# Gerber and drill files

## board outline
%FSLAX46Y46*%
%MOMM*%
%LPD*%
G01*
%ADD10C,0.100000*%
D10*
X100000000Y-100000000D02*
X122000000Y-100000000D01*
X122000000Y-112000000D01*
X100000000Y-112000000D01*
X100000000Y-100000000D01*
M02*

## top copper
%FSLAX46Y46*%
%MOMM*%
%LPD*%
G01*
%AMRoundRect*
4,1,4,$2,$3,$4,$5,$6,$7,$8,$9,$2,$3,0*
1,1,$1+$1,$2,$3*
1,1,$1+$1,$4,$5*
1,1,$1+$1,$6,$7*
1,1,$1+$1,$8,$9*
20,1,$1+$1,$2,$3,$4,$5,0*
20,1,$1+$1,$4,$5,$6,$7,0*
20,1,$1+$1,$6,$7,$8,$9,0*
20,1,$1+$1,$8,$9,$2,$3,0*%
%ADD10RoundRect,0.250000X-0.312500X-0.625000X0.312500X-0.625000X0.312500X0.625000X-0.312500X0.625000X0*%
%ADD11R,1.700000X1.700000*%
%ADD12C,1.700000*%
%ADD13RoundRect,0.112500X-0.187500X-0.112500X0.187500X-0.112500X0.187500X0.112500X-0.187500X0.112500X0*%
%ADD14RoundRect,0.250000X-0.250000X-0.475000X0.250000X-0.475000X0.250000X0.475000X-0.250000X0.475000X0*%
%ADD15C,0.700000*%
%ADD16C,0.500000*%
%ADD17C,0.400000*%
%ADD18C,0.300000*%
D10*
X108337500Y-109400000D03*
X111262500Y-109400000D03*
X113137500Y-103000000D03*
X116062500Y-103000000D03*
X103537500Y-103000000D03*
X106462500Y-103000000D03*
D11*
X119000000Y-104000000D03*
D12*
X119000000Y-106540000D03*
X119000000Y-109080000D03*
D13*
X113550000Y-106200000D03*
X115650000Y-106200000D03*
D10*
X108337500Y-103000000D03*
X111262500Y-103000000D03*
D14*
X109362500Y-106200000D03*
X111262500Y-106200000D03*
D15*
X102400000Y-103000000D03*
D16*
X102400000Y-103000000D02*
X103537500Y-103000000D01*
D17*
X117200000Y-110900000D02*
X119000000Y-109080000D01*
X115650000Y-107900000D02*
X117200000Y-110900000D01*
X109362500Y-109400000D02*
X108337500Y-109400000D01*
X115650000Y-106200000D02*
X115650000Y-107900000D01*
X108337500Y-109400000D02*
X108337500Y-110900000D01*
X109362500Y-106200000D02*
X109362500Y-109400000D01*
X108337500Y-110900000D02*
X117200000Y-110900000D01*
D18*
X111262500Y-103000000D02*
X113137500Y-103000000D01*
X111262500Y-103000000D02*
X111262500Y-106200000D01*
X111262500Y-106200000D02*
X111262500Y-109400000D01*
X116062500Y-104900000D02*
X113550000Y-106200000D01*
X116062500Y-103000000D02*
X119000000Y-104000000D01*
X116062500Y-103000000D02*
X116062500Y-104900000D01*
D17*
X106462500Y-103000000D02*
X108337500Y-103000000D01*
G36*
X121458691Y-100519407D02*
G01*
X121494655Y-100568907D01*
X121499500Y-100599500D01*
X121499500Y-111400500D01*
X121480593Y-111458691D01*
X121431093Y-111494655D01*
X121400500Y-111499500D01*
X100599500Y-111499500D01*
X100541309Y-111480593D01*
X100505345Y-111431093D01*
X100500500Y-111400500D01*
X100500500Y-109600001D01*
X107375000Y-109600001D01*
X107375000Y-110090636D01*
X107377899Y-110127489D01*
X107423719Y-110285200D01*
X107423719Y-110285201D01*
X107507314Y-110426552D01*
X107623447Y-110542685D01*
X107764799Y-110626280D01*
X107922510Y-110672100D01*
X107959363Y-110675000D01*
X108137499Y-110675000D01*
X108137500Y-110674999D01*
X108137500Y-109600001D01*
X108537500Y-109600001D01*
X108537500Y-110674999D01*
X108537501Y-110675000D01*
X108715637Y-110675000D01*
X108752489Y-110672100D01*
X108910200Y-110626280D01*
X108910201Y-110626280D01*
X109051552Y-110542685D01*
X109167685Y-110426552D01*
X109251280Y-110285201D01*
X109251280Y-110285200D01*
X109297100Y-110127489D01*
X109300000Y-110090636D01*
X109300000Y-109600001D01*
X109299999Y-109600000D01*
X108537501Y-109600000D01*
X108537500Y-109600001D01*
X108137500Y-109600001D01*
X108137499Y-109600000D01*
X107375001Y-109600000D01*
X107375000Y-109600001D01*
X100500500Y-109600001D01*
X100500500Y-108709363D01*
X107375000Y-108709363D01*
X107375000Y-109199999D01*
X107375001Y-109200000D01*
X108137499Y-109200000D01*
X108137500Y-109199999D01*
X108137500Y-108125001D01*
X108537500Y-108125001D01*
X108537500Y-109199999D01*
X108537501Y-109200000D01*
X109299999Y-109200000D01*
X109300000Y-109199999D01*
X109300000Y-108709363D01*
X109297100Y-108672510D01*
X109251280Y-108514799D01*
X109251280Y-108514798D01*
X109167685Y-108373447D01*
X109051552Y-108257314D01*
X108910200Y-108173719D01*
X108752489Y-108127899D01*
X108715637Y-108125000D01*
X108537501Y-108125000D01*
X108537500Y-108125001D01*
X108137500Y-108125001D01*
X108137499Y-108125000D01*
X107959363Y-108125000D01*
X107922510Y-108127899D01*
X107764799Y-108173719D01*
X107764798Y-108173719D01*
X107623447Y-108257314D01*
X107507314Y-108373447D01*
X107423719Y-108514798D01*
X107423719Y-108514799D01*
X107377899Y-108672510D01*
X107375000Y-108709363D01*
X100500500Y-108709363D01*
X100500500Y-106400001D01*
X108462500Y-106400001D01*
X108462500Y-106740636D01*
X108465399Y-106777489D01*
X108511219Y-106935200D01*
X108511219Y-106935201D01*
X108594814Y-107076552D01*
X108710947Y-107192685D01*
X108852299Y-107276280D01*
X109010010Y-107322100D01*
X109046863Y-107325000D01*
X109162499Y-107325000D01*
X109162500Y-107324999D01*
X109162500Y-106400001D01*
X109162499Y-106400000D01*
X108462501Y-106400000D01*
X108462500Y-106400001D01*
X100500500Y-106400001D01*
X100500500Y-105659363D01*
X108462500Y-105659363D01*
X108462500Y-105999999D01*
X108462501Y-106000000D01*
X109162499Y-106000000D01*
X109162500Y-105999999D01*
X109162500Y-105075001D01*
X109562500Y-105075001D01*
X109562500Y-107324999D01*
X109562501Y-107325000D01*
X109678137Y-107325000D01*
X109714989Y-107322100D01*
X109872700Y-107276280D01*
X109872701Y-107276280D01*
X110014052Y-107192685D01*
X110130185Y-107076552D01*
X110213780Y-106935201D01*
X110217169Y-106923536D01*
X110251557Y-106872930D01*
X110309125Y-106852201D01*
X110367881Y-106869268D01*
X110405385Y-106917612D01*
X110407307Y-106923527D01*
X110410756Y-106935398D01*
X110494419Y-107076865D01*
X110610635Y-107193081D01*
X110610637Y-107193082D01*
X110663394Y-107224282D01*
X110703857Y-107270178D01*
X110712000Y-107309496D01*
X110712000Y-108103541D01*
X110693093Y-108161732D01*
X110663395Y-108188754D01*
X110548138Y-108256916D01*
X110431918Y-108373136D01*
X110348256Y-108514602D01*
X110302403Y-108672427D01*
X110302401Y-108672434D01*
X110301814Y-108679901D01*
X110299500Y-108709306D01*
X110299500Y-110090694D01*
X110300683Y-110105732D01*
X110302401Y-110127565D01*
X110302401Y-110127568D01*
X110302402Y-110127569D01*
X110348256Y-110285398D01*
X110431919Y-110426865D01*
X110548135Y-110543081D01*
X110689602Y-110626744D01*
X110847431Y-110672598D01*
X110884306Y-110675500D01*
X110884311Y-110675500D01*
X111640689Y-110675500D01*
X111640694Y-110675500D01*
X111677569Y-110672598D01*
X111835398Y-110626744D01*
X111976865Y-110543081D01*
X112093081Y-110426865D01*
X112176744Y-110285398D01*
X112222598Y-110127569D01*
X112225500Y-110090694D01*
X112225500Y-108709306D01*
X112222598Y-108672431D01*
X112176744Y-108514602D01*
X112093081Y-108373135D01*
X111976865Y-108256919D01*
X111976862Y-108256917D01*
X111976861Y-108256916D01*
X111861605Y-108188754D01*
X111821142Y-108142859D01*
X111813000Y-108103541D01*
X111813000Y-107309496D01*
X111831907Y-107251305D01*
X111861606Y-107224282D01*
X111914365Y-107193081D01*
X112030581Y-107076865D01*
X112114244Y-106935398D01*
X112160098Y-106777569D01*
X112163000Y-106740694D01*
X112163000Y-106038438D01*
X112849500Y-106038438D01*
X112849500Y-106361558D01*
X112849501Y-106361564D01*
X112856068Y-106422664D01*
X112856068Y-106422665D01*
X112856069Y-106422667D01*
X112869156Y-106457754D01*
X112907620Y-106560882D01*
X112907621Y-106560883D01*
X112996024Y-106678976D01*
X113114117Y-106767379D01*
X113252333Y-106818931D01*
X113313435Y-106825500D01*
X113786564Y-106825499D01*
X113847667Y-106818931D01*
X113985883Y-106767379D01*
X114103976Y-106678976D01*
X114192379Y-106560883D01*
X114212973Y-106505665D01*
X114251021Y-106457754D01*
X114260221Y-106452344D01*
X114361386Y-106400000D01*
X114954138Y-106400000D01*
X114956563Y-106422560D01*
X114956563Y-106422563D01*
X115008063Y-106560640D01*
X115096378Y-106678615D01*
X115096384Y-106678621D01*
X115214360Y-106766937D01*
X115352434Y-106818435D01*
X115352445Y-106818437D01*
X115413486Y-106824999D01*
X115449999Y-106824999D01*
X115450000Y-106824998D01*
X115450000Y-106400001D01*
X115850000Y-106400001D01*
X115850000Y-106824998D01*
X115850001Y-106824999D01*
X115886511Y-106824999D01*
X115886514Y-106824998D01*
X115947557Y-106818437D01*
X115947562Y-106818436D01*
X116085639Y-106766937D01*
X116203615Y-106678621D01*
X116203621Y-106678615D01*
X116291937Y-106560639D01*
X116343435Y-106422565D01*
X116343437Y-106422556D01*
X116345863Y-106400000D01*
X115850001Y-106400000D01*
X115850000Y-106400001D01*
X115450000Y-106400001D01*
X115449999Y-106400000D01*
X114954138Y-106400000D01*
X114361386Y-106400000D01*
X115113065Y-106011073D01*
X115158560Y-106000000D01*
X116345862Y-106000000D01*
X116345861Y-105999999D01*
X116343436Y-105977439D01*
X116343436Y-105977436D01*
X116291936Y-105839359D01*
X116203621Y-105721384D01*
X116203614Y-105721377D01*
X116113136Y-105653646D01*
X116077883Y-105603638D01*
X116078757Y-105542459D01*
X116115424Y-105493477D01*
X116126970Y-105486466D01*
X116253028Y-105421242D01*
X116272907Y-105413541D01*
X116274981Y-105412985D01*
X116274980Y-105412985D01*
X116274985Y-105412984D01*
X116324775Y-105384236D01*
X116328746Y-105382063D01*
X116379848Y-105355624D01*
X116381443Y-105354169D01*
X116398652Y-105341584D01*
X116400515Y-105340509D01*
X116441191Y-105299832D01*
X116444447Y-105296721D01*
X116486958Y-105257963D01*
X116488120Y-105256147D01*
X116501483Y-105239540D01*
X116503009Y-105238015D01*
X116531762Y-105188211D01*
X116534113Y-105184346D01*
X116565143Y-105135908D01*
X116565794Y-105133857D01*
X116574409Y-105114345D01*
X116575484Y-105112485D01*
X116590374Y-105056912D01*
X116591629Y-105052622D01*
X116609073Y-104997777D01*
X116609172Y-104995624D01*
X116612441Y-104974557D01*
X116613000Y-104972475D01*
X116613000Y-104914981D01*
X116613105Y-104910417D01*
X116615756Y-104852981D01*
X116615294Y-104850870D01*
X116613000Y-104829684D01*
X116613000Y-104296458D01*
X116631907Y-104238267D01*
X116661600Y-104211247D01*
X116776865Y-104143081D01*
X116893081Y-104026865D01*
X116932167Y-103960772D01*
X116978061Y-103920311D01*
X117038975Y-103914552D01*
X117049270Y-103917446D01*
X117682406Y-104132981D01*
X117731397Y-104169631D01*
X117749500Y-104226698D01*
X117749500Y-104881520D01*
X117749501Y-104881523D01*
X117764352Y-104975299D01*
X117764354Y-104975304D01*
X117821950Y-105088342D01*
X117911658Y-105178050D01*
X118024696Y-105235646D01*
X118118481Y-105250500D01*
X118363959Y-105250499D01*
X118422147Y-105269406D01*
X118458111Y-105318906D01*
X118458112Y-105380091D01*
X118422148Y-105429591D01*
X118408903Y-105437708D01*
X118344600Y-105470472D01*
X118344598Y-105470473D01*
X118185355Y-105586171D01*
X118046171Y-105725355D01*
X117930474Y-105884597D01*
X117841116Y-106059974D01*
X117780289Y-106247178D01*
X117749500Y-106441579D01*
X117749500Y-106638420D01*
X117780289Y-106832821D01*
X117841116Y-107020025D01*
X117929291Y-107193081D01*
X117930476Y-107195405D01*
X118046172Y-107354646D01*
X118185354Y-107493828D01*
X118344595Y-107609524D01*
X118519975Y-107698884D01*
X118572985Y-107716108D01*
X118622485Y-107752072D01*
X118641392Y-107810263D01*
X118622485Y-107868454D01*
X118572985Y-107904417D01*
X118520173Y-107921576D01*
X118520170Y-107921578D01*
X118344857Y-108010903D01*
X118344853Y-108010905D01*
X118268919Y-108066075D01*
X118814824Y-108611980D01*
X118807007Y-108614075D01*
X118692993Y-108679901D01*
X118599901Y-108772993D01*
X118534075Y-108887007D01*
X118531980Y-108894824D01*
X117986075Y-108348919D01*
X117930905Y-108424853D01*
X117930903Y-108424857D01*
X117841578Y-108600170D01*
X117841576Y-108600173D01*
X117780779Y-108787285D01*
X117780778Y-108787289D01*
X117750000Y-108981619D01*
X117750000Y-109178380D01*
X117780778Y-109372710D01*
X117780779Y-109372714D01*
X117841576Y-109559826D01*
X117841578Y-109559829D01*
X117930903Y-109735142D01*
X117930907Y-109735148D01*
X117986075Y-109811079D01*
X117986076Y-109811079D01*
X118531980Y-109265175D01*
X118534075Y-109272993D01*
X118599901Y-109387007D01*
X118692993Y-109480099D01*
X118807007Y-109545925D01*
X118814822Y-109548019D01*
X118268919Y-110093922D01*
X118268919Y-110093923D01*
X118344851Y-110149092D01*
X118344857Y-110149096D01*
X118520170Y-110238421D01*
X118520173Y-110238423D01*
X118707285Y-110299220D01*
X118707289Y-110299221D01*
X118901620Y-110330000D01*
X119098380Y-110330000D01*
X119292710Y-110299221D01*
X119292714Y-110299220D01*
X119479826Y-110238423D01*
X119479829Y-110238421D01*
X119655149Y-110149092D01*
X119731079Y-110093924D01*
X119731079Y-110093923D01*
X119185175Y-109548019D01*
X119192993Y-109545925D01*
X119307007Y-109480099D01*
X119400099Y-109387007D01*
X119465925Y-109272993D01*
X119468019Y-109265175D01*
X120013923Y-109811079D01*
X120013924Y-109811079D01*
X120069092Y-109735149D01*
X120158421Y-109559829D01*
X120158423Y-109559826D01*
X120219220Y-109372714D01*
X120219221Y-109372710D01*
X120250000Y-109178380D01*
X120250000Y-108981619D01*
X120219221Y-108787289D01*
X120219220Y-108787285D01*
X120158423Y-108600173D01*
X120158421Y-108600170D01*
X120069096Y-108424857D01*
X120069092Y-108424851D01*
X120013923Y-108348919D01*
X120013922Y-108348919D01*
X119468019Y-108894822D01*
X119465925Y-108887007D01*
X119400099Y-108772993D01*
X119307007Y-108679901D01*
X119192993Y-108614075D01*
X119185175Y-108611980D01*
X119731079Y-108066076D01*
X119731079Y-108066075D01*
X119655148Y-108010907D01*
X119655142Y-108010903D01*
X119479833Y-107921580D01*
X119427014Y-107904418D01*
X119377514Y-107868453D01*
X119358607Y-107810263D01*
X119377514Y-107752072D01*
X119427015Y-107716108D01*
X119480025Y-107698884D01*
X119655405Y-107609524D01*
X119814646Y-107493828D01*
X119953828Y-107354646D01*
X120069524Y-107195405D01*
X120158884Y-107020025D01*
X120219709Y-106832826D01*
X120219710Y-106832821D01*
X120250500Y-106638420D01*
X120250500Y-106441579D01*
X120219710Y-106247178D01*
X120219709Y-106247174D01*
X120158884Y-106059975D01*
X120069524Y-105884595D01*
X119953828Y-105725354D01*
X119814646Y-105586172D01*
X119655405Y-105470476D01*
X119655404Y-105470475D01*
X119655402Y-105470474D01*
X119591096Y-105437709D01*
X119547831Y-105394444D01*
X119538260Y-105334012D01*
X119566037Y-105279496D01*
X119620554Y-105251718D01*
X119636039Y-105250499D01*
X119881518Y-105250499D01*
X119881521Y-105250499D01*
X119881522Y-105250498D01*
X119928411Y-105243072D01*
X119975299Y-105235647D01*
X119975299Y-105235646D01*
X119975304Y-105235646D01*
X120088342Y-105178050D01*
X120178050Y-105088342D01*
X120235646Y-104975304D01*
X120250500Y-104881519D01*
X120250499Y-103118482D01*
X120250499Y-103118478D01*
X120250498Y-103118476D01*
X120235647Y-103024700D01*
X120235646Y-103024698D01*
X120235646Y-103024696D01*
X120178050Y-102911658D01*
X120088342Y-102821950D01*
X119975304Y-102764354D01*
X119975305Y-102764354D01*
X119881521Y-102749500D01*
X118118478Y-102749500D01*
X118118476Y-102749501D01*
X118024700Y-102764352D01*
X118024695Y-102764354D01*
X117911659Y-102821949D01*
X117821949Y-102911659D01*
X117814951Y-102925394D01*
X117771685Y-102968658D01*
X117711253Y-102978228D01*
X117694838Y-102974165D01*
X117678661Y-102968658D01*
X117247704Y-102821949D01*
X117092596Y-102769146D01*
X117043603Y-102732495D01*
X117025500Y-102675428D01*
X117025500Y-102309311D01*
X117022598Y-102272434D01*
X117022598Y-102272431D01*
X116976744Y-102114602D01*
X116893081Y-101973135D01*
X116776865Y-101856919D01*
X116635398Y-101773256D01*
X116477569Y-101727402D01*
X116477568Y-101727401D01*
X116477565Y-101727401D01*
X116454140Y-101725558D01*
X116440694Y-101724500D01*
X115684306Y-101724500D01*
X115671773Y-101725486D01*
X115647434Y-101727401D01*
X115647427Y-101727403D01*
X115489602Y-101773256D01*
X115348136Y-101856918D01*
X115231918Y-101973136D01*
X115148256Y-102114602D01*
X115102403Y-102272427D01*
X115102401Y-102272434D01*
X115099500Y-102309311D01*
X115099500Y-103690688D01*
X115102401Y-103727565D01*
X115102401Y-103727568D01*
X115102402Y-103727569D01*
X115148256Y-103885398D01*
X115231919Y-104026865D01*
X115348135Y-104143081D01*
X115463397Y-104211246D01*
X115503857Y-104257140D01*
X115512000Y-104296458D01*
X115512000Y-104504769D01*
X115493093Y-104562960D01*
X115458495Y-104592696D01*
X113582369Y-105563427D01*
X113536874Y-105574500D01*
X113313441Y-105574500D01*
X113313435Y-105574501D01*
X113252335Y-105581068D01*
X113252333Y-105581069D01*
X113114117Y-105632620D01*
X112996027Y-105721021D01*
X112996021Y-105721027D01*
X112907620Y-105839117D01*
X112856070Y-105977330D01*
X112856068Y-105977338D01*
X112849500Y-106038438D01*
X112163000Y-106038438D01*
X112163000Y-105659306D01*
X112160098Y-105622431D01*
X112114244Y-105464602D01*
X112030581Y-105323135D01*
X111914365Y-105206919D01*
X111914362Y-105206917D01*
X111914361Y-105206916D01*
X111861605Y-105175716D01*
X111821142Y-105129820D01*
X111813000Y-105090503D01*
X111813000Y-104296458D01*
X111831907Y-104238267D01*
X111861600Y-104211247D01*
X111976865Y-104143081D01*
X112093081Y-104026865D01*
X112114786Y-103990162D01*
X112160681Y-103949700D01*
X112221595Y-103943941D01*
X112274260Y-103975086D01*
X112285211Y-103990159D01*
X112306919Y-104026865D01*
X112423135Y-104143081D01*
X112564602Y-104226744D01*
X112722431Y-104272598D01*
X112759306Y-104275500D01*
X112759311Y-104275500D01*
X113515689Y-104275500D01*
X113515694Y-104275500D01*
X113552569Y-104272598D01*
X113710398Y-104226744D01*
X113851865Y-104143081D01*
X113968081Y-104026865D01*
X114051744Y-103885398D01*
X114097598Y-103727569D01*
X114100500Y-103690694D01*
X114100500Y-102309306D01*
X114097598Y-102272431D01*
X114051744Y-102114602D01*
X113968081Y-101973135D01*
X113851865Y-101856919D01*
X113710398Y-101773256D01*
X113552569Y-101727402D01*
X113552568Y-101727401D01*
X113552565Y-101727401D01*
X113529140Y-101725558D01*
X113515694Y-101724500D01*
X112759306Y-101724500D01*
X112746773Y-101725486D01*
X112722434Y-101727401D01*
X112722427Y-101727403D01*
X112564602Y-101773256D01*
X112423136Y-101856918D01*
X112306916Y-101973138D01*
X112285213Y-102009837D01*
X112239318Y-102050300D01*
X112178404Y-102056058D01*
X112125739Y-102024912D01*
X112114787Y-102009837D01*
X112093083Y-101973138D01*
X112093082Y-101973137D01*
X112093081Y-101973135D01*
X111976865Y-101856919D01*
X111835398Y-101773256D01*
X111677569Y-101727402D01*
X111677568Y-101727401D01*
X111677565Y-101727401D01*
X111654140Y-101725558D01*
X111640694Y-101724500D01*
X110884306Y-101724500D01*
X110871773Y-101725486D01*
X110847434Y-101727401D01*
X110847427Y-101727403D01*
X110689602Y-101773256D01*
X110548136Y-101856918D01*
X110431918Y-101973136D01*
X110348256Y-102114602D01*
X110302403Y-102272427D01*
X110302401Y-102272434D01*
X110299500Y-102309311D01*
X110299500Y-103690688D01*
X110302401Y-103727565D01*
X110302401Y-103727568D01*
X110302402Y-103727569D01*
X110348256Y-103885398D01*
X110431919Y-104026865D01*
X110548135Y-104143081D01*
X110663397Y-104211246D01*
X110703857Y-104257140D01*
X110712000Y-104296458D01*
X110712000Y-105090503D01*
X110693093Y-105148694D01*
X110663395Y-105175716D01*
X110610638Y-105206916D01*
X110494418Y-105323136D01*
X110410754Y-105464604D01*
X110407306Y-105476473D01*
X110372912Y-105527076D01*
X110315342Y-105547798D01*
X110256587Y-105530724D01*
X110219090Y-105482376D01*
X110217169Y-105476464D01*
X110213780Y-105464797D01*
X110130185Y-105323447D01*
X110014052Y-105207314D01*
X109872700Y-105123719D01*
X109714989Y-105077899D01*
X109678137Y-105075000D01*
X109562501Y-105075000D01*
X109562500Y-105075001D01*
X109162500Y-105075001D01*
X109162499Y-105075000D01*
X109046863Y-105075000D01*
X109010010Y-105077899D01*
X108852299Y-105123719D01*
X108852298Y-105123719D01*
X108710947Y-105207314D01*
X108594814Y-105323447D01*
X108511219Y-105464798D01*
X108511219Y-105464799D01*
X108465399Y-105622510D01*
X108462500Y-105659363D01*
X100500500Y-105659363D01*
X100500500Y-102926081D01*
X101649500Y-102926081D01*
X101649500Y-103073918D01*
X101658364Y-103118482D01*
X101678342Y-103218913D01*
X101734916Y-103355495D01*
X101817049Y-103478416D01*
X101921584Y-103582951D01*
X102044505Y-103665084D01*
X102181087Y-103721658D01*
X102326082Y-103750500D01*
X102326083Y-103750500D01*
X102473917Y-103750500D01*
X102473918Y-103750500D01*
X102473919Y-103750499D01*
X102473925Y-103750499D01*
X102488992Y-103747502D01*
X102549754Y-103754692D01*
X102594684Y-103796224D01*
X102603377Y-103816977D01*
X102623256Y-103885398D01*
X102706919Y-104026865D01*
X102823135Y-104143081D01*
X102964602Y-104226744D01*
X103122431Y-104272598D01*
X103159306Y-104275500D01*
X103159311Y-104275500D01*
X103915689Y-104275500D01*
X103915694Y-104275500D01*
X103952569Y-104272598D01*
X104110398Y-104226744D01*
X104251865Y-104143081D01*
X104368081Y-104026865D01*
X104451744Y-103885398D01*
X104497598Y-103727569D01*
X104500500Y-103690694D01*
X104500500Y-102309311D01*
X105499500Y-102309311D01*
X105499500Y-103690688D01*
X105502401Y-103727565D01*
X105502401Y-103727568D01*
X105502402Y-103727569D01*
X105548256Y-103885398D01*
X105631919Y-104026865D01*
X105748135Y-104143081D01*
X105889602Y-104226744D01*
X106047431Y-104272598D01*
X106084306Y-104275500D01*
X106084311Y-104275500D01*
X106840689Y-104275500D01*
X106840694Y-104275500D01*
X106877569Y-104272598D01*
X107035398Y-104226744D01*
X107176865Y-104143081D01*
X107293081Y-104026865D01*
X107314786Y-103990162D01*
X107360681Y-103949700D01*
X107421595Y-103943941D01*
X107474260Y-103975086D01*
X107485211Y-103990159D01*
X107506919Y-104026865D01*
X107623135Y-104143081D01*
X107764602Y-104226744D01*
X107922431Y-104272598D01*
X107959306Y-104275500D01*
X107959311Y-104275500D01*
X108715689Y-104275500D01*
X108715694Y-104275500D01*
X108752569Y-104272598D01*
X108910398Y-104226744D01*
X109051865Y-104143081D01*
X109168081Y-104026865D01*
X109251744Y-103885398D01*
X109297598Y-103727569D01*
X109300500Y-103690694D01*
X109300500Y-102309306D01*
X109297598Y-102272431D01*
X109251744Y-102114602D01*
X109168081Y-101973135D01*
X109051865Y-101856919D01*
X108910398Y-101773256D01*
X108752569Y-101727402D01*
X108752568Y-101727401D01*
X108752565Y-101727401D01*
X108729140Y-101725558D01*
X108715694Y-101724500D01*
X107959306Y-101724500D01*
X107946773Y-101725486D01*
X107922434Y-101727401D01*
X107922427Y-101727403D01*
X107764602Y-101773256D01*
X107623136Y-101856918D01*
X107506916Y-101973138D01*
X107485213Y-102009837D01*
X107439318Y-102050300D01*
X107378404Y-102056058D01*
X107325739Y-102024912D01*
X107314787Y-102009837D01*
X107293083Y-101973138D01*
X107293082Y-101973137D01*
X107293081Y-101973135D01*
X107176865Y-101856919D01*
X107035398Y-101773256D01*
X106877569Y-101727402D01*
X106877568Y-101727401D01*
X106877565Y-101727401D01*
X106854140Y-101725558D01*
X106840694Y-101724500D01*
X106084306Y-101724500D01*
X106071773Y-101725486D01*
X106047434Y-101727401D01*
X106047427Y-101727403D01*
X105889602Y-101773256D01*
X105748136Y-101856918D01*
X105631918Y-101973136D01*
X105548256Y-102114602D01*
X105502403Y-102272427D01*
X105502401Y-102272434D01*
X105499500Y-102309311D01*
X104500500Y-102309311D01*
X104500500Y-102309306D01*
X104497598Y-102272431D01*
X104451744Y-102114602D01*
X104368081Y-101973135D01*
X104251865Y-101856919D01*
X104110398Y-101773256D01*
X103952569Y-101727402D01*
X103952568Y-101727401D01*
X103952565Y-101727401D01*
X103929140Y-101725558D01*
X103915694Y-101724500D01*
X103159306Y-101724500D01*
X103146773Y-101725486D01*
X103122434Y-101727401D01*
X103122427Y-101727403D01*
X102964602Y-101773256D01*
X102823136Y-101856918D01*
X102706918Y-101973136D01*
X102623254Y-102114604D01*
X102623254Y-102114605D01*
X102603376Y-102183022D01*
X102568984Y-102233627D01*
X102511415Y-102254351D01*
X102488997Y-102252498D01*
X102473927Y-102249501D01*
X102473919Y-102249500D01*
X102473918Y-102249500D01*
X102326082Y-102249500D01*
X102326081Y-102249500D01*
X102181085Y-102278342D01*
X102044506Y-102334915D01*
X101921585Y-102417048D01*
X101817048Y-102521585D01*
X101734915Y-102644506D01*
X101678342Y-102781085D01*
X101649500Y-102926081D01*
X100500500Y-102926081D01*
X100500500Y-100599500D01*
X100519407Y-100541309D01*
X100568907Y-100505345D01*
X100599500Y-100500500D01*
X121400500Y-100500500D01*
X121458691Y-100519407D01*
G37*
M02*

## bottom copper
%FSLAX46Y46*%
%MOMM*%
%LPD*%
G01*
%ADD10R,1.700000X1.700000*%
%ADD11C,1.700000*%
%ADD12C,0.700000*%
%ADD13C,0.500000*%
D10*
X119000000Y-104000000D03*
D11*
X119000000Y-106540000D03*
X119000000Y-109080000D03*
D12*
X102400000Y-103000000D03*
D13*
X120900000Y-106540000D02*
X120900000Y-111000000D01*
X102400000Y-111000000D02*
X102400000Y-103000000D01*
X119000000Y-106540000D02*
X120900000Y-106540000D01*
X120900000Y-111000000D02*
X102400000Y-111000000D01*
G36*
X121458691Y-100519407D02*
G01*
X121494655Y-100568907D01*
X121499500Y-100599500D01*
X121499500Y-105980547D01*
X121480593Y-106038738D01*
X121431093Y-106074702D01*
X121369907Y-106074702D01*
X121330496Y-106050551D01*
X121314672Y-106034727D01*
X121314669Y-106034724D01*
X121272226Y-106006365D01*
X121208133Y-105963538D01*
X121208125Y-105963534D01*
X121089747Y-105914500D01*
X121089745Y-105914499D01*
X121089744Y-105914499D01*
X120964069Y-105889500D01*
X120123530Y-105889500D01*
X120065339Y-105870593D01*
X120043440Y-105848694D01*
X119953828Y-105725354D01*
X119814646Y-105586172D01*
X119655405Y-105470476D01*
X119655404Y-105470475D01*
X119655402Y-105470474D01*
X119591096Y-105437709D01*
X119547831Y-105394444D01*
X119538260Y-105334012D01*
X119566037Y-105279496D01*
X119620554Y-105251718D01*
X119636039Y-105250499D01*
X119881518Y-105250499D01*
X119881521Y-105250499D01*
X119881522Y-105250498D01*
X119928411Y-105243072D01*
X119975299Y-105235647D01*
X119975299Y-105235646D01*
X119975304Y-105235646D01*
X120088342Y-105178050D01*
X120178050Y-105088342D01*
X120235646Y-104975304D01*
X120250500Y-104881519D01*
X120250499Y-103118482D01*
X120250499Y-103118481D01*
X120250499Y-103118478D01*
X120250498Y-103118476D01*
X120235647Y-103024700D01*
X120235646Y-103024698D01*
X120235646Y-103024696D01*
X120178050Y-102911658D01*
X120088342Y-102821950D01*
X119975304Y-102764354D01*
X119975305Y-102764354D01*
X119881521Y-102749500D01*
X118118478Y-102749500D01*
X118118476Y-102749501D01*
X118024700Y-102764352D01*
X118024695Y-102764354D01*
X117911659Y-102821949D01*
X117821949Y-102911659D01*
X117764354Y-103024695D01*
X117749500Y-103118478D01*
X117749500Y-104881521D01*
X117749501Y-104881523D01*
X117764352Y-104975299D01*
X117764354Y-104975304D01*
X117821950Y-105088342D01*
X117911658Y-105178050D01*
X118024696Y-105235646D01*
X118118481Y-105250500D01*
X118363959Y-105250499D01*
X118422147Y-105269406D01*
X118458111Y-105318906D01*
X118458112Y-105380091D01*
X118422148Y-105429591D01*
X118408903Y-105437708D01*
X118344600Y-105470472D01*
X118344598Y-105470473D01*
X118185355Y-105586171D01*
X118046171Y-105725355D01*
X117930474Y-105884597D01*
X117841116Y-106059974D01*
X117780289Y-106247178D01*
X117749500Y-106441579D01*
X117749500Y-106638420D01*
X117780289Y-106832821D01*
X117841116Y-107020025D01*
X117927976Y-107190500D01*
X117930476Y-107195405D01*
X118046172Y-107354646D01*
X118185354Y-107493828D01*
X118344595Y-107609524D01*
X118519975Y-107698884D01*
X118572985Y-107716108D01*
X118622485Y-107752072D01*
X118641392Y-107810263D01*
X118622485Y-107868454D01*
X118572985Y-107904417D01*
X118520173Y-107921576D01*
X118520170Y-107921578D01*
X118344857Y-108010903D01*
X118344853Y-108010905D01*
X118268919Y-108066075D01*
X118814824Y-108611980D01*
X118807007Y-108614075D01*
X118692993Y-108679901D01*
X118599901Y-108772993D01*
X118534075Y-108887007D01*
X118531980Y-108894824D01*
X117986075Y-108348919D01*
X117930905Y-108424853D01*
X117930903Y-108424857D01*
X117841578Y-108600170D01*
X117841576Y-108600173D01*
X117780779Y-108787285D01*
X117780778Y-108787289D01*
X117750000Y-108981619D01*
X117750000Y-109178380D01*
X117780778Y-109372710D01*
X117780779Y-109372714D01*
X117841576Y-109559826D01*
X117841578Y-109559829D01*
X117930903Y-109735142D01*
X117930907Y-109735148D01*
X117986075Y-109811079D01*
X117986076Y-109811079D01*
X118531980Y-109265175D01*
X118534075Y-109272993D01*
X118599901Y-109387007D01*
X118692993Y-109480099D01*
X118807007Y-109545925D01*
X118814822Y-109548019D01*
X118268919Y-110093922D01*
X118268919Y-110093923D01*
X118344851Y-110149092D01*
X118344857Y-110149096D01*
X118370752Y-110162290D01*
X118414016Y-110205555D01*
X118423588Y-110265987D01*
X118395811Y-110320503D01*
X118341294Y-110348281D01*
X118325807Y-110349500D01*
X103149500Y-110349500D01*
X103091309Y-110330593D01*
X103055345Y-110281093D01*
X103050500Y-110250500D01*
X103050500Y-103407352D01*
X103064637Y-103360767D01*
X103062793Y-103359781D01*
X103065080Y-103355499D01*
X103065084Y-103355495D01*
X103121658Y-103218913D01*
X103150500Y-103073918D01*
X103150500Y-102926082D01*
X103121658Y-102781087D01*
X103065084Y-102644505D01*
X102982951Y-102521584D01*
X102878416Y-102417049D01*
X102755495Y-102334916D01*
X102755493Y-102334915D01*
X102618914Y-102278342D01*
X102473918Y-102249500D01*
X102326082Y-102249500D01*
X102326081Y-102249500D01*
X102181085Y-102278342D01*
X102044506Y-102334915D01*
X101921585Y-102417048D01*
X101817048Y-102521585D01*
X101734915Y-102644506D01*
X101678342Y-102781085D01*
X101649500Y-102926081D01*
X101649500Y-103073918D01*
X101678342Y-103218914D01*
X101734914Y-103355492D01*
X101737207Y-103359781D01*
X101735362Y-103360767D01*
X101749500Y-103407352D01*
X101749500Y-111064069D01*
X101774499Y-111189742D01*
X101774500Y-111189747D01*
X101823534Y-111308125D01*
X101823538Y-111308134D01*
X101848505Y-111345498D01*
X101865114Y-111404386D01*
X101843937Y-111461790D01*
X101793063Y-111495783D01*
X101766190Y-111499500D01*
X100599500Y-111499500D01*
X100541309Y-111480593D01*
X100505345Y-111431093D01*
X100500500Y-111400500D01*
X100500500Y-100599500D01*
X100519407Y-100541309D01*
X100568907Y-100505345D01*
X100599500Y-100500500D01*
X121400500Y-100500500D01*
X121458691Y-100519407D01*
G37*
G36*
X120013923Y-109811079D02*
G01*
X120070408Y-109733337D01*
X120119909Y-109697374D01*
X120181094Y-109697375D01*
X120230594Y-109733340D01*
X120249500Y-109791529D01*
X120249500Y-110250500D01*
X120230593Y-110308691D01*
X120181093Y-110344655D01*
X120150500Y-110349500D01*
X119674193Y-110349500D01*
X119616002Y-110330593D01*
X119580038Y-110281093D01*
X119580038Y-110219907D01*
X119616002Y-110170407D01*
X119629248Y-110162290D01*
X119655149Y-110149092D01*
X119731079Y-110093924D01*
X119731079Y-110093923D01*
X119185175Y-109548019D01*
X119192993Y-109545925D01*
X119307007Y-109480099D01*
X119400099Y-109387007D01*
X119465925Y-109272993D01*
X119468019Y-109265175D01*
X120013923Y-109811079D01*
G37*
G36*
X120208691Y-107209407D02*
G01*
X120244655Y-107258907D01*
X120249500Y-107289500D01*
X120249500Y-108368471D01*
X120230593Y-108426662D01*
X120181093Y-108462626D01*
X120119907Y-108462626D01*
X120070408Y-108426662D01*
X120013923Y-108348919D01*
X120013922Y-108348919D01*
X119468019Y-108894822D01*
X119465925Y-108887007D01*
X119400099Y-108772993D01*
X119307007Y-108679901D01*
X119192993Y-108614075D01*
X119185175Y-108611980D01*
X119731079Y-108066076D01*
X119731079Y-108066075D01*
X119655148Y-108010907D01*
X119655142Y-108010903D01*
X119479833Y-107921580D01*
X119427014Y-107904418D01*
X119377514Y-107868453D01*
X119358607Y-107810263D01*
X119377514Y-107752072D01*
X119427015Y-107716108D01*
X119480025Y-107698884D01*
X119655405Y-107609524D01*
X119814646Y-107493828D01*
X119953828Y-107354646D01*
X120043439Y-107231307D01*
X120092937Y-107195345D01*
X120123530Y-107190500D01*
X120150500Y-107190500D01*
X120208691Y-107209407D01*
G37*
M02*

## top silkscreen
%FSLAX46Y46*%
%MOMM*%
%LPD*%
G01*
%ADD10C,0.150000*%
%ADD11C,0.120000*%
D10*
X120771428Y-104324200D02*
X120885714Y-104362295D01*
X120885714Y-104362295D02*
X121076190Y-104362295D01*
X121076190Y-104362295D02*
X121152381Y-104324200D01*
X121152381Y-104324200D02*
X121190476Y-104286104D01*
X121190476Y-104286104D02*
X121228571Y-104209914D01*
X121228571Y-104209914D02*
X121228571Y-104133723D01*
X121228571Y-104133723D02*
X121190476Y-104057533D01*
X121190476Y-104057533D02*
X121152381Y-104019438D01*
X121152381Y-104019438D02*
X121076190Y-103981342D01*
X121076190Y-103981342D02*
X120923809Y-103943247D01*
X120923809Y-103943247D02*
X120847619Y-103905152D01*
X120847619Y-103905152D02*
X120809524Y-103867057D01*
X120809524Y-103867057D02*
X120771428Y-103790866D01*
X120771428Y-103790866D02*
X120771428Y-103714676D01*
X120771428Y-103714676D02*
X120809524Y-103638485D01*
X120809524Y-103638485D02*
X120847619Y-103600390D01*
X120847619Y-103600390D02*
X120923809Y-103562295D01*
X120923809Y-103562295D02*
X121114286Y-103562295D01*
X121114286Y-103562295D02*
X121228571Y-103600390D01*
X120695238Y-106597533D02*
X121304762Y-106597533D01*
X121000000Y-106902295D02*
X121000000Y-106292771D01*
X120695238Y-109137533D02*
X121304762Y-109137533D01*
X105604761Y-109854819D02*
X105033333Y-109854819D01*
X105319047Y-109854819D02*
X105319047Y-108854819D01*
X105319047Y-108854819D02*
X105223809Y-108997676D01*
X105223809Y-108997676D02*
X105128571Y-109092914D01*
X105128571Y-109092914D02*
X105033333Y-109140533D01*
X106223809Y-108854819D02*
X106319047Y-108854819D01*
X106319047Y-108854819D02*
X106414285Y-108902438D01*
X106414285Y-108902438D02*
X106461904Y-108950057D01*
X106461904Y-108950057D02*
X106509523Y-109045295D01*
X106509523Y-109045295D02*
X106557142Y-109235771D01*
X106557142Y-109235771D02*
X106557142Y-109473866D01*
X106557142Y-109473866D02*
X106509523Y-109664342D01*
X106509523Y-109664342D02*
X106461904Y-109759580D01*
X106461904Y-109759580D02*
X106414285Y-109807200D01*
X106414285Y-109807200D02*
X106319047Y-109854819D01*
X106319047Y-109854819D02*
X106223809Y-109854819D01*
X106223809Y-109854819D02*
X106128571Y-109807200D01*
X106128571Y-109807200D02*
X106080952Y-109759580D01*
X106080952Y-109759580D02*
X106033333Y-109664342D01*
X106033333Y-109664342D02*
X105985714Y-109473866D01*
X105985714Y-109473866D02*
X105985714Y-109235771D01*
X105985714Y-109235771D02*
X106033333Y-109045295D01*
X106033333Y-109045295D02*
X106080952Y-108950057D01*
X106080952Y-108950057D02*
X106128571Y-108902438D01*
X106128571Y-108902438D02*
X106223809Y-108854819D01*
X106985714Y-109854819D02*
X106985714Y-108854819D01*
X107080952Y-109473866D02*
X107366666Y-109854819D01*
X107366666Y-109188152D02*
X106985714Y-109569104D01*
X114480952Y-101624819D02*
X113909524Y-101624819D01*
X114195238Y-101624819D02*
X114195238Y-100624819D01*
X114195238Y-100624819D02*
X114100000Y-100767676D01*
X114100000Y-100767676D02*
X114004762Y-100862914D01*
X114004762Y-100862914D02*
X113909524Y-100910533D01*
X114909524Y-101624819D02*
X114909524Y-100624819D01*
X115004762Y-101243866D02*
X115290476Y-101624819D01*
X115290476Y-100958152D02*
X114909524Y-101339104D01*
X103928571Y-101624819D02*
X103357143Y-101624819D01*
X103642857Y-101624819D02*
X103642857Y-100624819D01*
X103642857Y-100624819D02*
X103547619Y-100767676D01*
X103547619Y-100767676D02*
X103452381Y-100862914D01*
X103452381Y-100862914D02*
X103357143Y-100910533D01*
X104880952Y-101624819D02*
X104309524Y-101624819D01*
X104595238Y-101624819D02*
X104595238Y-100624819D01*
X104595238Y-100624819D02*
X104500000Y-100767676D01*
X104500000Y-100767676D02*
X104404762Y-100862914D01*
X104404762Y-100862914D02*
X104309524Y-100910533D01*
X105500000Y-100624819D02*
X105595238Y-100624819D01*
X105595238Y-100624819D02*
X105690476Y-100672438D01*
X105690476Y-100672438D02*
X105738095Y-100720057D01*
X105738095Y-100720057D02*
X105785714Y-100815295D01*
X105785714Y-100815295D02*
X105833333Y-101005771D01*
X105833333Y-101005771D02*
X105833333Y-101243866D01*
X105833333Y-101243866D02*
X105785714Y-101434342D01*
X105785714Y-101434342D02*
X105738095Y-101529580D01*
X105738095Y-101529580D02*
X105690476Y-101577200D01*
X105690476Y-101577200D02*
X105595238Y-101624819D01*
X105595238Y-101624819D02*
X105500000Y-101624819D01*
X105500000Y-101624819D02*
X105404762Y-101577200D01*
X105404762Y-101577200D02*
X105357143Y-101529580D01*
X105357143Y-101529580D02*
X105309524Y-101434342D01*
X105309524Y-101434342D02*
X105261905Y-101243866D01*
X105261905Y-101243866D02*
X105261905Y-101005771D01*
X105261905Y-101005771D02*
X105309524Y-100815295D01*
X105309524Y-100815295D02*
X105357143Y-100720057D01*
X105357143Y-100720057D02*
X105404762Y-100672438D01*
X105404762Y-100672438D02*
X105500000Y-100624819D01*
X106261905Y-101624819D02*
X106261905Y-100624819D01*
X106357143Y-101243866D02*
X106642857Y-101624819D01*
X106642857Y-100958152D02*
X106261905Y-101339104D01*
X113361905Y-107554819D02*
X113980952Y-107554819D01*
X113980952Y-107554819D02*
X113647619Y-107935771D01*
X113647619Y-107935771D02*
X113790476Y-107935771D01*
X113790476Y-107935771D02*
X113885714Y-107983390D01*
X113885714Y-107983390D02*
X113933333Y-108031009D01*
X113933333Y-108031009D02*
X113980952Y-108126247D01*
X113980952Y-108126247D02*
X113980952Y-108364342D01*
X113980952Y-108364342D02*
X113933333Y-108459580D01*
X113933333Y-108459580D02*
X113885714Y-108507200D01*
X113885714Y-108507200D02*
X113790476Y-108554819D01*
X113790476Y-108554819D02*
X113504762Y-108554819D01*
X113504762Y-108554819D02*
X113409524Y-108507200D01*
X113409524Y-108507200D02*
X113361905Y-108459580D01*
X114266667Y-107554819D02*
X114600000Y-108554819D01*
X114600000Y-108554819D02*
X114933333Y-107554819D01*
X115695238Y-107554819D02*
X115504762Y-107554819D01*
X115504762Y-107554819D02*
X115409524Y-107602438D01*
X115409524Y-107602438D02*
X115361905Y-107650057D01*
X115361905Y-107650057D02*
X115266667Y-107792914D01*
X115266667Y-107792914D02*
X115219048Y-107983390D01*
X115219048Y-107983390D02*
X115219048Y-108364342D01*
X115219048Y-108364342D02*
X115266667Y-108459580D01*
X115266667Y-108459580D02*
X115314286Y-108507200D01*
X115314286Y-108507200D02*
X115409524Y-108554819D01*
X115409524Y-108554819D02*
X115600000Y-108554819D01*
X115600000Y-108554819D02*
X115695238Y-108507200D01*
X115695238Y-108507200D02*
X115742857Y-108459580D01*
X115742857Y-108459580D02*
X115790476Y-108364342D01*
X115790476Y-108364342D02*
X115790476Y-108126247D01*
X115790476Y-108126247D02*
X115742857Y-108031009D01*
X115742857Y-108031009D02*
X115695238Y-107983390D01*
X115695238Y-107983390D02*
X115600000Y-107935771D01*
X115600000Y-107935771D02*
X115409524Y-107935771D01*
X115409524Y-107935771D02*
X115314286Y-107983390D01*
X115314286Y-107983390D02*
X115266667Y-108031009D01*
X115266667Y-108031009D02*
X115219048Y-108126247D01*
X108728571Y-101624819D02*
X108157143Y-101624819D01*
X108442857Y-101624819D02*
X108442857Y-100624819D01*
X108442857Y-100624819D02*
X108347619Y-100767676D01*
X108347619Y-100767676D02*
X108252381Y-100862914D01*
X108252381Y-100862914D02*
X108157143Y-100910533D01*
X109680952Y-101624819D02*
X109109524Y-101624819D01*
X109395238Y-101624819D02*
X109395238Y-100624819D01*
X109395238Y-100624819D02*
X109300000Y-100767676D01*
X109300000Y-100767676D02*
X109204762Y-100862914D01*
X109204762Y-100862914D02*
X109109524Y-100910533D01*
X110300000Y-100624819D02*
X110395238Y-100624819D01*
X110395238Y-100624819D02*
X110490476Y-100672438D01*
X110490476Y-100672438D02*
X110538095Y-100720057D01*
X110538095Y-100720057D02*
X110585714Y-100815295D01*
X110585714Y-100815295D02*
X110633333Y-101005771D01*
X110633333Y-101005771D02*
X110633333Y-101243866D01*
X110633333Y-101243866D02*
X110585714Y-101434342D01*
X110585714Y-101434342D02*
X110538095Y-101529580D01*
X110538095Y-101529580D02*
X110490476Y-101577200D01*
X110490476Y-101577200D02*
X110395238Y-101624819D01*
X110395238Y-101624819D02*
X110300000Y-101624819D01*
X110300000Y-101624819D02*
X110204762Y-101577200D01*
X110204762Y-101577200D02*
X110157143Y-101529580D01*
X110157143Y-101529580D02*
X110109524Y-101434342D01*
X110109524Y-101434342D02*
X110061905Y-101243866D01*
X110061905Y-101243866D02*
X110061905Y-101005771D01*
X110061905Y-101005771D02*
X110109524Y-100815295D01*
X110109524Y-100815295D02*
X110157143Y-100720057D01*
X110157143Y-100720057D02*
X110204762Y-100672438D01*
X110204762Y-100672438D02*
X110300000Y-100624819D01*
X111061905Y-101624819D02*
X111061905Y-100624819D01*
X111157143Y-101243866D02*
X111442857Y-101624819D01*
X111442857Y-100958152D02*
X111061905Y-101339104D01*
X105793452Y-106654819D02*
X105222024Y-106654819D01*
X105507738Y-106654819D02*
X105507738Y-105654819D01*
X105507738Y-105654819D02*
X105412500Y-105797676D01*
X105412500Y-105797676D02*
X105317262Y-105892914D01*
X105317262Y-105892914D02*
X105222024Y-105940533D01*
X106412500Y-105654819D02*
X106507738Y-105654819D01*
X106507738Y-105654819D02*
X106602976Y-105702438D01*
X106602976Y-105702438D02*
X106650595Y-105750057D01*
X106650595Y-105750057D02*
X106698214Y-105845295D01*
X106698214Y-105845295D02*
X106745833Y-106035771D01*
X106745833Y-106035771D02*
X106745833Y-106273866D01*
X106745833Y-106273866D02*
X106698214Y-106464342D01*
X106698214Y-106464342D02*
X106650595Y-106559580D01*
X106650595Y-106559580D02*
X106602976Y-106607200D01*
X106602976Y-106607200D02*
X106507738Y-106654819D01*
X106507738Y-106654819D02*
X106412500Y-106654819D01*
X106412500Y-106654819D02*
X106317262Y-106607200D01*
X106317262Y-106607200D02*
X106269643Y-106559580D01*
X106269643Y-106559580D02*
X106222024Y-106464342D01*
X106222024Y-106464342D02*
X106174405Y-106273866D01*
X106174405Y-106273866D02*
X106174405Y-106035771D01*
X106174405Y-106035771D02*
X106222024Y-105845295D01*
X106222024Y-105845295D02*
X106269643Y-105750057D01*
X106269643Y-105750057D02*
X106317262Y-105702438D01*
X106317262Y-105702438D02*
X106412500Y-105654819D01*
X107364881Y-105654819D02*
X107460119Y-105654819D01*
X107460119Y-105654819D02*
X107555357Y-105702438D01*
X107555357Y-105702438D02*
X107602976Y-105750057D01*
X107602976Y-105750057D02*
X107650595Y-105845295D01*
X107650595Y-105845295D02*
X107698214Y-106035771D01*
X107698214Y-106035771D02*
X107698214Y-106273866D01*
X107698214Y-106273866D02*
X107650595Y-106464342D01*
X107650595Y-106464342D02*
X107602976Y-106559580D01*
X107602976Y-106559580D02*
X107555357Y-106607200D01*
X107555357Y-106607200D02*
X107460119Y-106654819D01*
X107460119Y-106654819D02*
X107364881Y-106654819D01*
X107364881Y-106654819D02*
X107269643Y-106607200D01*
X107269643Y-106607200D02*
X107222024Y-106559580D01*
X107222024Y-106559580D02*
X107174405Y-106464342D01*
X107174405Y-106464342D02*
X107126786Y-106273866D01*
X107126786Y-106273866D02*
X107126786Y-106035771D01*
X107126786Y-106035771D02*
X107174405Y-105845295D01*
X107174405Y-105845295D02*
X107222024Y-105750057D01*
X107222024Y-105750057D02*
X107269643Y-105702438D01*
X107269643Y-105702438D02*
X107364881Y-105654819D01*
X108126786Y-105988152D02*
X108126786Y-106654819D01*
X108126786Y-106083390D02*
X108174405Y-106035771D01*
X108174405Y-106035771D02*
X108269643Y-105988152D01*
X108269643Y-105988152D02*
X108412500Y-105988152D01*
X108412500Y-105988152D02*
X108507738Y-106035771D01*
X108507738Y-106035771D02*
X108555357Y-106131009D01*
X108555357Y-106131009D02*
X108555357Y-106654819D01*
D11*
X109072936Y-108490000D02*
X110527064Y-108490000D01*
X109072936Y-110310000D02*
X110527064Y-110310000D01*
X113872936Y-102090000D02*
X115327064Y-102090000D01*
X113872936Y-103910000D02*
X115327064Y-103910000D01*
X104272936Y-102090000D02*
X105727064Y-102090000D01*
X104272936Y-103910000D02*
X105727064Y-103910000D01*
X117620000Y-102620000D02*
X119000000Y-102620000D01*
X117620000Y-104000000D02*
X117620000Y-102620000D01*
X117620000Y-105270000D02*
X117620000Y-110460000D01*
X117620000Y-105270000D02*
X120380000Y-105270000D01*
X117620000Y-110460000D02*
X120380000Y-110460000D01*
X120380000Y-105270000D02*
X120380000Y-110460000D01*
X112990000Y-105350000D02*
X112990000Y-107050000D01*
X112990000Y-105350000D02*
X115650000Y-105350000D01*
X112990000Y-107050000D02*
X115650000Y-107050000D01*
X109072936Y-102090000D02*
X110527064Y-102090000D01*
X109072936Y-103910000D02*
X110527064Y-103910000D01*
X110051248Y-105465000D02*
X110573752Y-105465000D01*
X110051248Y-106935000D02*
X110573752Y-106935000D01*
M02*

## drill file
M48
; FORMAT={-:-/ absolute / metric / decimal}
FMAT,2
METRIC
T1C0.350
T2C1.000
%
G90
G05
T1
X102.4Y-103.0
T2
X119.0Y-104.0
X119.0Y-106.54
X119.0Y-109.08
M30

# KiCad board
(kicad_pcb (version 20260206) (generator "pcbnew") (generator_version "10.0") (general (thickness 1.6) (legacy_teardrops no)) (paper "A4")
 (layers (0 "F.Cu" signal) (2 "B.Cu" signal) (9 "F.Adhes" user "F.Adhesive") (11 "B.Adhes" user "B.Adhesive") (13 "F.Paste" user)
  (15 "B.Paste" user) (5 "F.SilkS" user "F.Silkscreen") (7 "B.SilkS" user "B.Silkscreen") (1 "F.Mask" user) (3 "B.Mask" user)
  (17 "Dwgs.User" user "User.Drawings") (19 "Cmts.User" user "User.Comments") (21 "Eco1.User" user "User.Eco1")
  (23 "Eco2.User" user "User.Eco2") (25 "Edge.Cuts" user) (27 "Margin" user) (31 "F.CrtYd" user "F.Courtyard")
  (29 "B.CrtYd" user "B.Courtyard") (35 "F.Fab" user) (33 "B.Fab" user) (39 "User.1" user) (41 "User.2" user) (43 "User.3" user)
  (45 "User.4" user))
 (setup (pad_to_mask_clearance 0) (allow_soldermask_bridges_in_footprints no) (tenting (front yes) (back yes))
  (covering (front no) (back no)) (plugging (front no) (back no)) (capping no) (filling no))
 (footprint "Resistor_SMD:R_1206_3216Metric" (layer "F.Cu") (at 109.8 109.4)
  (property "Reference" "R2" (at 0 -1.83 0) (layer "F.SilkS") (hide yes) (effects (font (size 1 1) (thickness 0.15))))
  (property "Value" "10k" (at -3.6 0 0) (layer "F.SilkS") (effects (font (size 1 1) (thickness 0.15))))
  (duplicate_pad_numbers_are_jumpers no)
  (fp_line (start -0.727064 -0.91) (end 0.727064 -0.91) (stroke (width 0.12) (type solid)) (layer "F.SilkS"))
  (fp_line (start -0.727064 0.91) (end 0.727064 0.91) (stroke (width 0.12) (type solid)) (layer "F.SilkS"))
  (pad "1" smd roundrect (at -1.4625 0) (size 1.125 1.75) (layers "F.Cu" "F.Mask" "F.Paste") (roundrect_rratio 0.222222) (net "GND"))
  (pad "2" smd roundrect (at 1.4625 0) (size 1.125 1.75) (layers "F.Cu" "F.Mask" "F.Paste") (roundrect_rratio 0.222222) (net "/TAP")))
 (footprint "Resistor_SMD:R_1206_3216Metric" (layer "F.Cu") (at 114.6 103)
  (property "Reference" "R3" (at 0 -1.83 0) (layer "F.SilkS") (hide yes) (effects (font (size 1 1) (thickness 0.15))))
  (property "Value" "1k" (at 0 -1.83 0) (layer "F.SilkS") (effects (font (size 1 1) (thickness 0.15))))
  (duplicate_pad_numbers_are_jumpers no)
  (fp_line (start -0.727064 -0.91) (end 0.727064 -0.91) (stroke (width 0.12) (type solid)) (layer "F.SilkS"))
  (fp_line (start -0.727064 0.91) (end 0.727064 0.91) (stroke (width 0.12) (type solid)) (layer "F.SilkS"))
  (pad "1" smd roundrect (at -1.4625 0) (size 1.125 1.75) (layers "F.Cu" "F.Mask" "F.Paste") (roundrect_rratio 0.222222) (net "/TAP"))
  (pad "2" smd roundrect (at 1.4625 0) (size 1.125 1.75) (layers "F.Cu" "F.Mask" "F.Paste") (roundrect_rratio 0.222222) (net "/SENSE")))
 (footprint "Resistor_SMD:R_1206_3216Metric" (layer "F.Cu") (at 105 103)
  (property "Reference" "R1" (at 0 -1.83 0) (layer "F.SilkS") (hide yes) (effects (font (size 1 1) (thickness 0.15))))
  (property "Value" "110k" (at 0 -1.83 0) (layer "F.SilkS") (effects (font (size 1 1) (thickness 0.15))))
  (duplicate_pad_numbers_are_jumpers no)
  (fp_line (start -0.727064 -0.91) (end 0.727064 -0.91) (stroke (width 0.12) (type solid)) (layer "F.SilkS"))
  (fp_line (start -0.727064 0.91) (end 0.727064 0.91) (stroke (width 0.12) (type solid)) (layer "F.SilkS"))
  (pad "1" smd roundrect (at -1.4625 0) (size 1.125 1.75) (layers "F.Cu" "F.Mask" "F.Paste") (roundrect_rratio 0.222222) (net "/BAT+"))
  (pad "2" smd roundrect (at 1.4625 0) (size 1.125 1.75) (layers "F.Cu" "F.Mask" "F.Paste") (roundrect_rratio 0.222222) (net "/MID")))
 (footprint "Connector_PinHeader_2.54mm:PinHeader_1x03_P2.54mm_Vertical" (layer "F.Cu") (at 119 104)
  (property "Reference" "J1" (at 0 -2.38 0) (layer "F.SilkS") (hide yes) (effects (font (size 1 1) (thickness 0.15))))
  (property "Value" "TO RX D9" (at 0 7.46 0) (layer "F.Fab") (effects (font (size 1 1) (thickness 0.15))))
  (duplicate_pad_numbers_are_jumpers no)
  (fp_line (start -1.38 -1.38) (end 0 -1.38) (stroke (width 0.12) (type solid)) (layer "F.SilkS"))
  (fp_line (start -1.38 0) (end -1.38 -1.38) (stroke (width 0.12) (type solid)) (layer "F.SilkS"))
  (fp_line (start -1.38 1.27) (end -1.38 6.46) (stroke (width 0.12) (type solid)) (layer "F.SilkS"))
  (fp_line (start -1.38 1.27) (end 1.38 1.27) (stroke (width 0.12) (type solid)) (layer "F.SilkS"))
  (fp_line (start -1.38 6.46) (end 1.38 6.46) (stroke (width 0.12) (type solid)) (layer "F.SilkS"))
  (fp_line (start 1.38 1.27) (end 1.38 6.46) (stroke (width 0.12) (type solid)) (layer "F.SilkS"))
  (pad "1" thru_hole rect (at 0 0) (size 1.7 1.7) (drill 1) (layers "*.Cu" "*.Mask") (remove_unused_layers no) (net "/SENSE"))
  (pad "2" thru_hole circle (at 0 2.54) (size 1.7 1.7) (drill 1) (layers "*.Cu" "*.Mask") (remove_unused_layers no) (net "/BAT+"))
  (pad "3" thru_hole circle (at 0 5.08) (size 1.7 1.7) (drill 1) (layers "*.Cu" "*.Mask") (remove_unused_layers no) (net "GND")))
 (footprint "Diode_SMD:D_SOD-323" (layer "F.Cu") (at 114.6 106.2)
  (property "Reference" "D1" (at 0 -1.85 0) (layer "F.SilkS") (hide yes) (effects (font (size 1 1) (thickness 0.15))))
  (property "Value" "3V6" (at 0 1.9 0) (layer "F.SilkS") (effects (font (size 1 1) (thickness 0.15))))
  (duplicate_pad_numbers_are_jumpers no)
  (fp_line (start -1.61 -0.85) (end -1.61 0.85) (stroke (width 0.12) (type solid)) (layer "F.SilkS"))
  (fp_line (start -1.61 -0.85) (end 1.05 -0.85) (stroke (width 0.12) (type solid)) (layer "F.SilkS"))
  (fp_line (start -1.61 0.85) (end 1.05 0.85) (stroke (width 0.12) (type solid)) (layer "F.SilkS"))
  (pad "1" smd roundrect (at -1.05 0) (size 0.6 0.45) (layers "F.Cu" "F.Mask" "F.Paste") (roundrect_rratio 0.25) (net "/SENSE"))
  (pad "2" smd roundrect (at 1.05 0) (size 0.6 0.45) (layers "F.Cu" "F.Mask" "F.Paste") (roundrect_rratio 0.25) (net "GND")))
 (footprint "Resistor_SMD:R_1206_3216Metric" (layer "F.Cu") (at 109.8 103)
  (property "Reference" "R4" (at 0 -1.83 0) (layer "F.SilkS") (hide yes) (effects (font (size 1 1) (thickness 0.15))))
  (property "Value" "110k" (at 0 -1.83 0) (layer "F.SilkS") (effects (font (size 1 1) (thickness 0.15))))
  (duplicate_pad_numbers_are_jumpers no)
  (fp_line (start -0.727064 -0.91) (end 0.727064 -0.91) (stroke (width 0.12) (type solid)) (layer "F.SilkS"))
  (fp_line (start -0.727064 0.91) (end 0.727064 0.91) (stroke (width 0.12) (type solid)) (layer "F.SilkS"))
  (pad "1" smd roundrect (at -1.4625 0) (size 1.125 1.75) (layers "F.Cu" "F.Mask" "F.Paste") (roundrect_rratio 0.222222) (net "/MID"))
  (pad "2" smd roundrect (at 1.4625 0) (size 1.125 1.75) (layers "F.Cu" "F.Mask" "F.Paste") (roundrect_rratio 0.222222) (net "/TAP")))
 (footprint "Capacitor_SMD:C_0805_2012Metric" (layer "F.Cu") (at 110.3125 106.2)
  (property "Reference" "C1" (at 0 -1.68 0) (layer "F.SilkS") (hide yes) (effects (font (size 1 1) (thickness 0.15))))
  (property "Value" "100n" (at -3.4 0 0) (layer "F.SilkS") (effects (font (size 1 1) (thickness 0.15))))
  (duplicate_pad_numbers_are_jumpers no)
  (fp_line (start -0.261252 -0.735) (end 0.261252 -0.735) (stroke (width 0.12) (type solid)) (layer "F.SilkS"))
  (fp_line (start -0.261252 0.735) (end 0.261252 0.735) (stroke (width 0.12) (type solid)) (layer "F.SilkS"))
  (pad "1" smd roundrect (at -0.95 0) (size 1 1.45) (layers "F.Cu" "F.Mask" "F.Paste") (roundrect_rratio 0.25) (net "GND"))
  (pad "2" smd roundrect (at 0.95 0) (size 1 1.45) (layers "F.Cu" "F.Mask" "F.Paste") (roundrect_rratio 0.25) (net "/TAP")))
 (gr_rect (start 100 100) (end 122 112) (stroke (width 0.1) (type solid)) (fill no) (layer "Edge.Cuts"))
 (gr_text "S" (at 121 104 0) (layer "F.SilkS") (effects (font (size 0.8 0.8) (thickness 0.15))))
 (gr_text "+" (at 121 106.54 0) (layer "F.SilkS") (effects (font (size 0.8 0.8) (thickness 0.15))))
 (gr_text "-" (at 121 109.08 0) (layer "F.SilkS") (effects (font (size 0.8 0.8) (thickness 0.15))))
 (segment (start 102.4 103) (end 103.5375 103) (width 0.5) (layer "F.Cu") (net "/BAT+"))
 (via (at 102.4 103) (size 0.7) (drill 0.35) (layers "F.Cu" "B.Cu") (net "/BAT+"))
 (segment (start 120.9 106.54) (end 120.9 111) (width 0.5) (layer "B.Cu") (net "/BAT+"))
 (segment (start 102.4 111) (end 102.4 103) (width 0.5) (layer "B.Cu") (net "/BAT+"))
 (segment (start 119 106.54) (end 120.9 106.54) (width 0.5) (layer "B.Cu") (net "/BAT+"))
 (segment (start 120.9 111) (end 102.4 111) (width 0.5) (layer "B.Cu") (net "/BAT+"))
 (segment (start 117.2 110.9) (end 119 109.08) (width 0.4) (layer "F.Cu") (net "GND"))
 (segment (start 115.65 107.9) (end 117.2 110.9) (width 0.4) (layer "F.Cu") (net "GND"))
 (segment (start 109.3625 109.4) (end 108.3375 109.4) (width 0.4) (layer "F.Cu") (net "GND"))
 (segment (start 115.65 106.2) (end 115.65 107.9) (width 0.4) (layer "F.Cu") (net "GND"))
 (segment (start 108.3375 109.4) (end 108.3375 110.9) (width 0.4) (layer "F.Cu") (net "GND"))
 (segment (start 109.3625 106.2) (end 109.3625 109.4) (width 0.4) (layer "F.Cu") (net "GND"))
 (segment (start 108.3375 110.9) (end 117.2 110.9) (width 0.4) (layer "F.Cu") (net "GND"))
 (segment (start 111.2625 103) (end 113.1375 103) (width 0.3) (layer "F.Cu") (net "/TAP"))
 (segment (start 111.2625 103) (end 111.2625 106.2) (width 0.3) (layer "F.Cu") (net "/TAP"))
 (segment (start 111.2625 106.2) (end 111.2625 109.4) (width 0.3) (layer "F.Cu") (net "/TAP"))
 (segment (start 116.0625 104.9) (end 113.55 106.2) (width 0.3) (layer "F.Cu") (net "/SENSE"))
 (segment (start 116.0625 103) (end 119 104) (width 0.3) (layer "F.Cu") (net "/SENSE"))
 (segment (start 116.0625 103) (end 116.0625 104.9) (width 0.3) (layer "F.Cu") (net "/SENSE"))
 (segment (start 106.4625 103) (end 108.3375 103) (width 0.4) (layer "F.Cu") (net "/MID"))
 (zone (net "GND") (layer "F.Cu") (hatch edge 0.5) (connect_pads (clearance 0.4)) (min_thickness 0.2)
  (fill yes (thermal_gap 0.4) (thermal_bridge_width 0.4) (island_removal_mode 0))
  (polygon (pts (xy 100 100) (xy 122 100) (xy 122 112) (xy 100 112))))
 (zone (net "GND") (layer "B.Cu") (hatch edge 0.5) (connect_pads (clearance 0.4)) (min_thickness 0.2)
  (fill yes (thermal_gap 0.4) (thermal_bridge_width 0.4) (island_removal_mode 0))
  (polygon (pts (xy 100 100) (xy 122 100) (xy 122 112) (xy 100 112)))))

